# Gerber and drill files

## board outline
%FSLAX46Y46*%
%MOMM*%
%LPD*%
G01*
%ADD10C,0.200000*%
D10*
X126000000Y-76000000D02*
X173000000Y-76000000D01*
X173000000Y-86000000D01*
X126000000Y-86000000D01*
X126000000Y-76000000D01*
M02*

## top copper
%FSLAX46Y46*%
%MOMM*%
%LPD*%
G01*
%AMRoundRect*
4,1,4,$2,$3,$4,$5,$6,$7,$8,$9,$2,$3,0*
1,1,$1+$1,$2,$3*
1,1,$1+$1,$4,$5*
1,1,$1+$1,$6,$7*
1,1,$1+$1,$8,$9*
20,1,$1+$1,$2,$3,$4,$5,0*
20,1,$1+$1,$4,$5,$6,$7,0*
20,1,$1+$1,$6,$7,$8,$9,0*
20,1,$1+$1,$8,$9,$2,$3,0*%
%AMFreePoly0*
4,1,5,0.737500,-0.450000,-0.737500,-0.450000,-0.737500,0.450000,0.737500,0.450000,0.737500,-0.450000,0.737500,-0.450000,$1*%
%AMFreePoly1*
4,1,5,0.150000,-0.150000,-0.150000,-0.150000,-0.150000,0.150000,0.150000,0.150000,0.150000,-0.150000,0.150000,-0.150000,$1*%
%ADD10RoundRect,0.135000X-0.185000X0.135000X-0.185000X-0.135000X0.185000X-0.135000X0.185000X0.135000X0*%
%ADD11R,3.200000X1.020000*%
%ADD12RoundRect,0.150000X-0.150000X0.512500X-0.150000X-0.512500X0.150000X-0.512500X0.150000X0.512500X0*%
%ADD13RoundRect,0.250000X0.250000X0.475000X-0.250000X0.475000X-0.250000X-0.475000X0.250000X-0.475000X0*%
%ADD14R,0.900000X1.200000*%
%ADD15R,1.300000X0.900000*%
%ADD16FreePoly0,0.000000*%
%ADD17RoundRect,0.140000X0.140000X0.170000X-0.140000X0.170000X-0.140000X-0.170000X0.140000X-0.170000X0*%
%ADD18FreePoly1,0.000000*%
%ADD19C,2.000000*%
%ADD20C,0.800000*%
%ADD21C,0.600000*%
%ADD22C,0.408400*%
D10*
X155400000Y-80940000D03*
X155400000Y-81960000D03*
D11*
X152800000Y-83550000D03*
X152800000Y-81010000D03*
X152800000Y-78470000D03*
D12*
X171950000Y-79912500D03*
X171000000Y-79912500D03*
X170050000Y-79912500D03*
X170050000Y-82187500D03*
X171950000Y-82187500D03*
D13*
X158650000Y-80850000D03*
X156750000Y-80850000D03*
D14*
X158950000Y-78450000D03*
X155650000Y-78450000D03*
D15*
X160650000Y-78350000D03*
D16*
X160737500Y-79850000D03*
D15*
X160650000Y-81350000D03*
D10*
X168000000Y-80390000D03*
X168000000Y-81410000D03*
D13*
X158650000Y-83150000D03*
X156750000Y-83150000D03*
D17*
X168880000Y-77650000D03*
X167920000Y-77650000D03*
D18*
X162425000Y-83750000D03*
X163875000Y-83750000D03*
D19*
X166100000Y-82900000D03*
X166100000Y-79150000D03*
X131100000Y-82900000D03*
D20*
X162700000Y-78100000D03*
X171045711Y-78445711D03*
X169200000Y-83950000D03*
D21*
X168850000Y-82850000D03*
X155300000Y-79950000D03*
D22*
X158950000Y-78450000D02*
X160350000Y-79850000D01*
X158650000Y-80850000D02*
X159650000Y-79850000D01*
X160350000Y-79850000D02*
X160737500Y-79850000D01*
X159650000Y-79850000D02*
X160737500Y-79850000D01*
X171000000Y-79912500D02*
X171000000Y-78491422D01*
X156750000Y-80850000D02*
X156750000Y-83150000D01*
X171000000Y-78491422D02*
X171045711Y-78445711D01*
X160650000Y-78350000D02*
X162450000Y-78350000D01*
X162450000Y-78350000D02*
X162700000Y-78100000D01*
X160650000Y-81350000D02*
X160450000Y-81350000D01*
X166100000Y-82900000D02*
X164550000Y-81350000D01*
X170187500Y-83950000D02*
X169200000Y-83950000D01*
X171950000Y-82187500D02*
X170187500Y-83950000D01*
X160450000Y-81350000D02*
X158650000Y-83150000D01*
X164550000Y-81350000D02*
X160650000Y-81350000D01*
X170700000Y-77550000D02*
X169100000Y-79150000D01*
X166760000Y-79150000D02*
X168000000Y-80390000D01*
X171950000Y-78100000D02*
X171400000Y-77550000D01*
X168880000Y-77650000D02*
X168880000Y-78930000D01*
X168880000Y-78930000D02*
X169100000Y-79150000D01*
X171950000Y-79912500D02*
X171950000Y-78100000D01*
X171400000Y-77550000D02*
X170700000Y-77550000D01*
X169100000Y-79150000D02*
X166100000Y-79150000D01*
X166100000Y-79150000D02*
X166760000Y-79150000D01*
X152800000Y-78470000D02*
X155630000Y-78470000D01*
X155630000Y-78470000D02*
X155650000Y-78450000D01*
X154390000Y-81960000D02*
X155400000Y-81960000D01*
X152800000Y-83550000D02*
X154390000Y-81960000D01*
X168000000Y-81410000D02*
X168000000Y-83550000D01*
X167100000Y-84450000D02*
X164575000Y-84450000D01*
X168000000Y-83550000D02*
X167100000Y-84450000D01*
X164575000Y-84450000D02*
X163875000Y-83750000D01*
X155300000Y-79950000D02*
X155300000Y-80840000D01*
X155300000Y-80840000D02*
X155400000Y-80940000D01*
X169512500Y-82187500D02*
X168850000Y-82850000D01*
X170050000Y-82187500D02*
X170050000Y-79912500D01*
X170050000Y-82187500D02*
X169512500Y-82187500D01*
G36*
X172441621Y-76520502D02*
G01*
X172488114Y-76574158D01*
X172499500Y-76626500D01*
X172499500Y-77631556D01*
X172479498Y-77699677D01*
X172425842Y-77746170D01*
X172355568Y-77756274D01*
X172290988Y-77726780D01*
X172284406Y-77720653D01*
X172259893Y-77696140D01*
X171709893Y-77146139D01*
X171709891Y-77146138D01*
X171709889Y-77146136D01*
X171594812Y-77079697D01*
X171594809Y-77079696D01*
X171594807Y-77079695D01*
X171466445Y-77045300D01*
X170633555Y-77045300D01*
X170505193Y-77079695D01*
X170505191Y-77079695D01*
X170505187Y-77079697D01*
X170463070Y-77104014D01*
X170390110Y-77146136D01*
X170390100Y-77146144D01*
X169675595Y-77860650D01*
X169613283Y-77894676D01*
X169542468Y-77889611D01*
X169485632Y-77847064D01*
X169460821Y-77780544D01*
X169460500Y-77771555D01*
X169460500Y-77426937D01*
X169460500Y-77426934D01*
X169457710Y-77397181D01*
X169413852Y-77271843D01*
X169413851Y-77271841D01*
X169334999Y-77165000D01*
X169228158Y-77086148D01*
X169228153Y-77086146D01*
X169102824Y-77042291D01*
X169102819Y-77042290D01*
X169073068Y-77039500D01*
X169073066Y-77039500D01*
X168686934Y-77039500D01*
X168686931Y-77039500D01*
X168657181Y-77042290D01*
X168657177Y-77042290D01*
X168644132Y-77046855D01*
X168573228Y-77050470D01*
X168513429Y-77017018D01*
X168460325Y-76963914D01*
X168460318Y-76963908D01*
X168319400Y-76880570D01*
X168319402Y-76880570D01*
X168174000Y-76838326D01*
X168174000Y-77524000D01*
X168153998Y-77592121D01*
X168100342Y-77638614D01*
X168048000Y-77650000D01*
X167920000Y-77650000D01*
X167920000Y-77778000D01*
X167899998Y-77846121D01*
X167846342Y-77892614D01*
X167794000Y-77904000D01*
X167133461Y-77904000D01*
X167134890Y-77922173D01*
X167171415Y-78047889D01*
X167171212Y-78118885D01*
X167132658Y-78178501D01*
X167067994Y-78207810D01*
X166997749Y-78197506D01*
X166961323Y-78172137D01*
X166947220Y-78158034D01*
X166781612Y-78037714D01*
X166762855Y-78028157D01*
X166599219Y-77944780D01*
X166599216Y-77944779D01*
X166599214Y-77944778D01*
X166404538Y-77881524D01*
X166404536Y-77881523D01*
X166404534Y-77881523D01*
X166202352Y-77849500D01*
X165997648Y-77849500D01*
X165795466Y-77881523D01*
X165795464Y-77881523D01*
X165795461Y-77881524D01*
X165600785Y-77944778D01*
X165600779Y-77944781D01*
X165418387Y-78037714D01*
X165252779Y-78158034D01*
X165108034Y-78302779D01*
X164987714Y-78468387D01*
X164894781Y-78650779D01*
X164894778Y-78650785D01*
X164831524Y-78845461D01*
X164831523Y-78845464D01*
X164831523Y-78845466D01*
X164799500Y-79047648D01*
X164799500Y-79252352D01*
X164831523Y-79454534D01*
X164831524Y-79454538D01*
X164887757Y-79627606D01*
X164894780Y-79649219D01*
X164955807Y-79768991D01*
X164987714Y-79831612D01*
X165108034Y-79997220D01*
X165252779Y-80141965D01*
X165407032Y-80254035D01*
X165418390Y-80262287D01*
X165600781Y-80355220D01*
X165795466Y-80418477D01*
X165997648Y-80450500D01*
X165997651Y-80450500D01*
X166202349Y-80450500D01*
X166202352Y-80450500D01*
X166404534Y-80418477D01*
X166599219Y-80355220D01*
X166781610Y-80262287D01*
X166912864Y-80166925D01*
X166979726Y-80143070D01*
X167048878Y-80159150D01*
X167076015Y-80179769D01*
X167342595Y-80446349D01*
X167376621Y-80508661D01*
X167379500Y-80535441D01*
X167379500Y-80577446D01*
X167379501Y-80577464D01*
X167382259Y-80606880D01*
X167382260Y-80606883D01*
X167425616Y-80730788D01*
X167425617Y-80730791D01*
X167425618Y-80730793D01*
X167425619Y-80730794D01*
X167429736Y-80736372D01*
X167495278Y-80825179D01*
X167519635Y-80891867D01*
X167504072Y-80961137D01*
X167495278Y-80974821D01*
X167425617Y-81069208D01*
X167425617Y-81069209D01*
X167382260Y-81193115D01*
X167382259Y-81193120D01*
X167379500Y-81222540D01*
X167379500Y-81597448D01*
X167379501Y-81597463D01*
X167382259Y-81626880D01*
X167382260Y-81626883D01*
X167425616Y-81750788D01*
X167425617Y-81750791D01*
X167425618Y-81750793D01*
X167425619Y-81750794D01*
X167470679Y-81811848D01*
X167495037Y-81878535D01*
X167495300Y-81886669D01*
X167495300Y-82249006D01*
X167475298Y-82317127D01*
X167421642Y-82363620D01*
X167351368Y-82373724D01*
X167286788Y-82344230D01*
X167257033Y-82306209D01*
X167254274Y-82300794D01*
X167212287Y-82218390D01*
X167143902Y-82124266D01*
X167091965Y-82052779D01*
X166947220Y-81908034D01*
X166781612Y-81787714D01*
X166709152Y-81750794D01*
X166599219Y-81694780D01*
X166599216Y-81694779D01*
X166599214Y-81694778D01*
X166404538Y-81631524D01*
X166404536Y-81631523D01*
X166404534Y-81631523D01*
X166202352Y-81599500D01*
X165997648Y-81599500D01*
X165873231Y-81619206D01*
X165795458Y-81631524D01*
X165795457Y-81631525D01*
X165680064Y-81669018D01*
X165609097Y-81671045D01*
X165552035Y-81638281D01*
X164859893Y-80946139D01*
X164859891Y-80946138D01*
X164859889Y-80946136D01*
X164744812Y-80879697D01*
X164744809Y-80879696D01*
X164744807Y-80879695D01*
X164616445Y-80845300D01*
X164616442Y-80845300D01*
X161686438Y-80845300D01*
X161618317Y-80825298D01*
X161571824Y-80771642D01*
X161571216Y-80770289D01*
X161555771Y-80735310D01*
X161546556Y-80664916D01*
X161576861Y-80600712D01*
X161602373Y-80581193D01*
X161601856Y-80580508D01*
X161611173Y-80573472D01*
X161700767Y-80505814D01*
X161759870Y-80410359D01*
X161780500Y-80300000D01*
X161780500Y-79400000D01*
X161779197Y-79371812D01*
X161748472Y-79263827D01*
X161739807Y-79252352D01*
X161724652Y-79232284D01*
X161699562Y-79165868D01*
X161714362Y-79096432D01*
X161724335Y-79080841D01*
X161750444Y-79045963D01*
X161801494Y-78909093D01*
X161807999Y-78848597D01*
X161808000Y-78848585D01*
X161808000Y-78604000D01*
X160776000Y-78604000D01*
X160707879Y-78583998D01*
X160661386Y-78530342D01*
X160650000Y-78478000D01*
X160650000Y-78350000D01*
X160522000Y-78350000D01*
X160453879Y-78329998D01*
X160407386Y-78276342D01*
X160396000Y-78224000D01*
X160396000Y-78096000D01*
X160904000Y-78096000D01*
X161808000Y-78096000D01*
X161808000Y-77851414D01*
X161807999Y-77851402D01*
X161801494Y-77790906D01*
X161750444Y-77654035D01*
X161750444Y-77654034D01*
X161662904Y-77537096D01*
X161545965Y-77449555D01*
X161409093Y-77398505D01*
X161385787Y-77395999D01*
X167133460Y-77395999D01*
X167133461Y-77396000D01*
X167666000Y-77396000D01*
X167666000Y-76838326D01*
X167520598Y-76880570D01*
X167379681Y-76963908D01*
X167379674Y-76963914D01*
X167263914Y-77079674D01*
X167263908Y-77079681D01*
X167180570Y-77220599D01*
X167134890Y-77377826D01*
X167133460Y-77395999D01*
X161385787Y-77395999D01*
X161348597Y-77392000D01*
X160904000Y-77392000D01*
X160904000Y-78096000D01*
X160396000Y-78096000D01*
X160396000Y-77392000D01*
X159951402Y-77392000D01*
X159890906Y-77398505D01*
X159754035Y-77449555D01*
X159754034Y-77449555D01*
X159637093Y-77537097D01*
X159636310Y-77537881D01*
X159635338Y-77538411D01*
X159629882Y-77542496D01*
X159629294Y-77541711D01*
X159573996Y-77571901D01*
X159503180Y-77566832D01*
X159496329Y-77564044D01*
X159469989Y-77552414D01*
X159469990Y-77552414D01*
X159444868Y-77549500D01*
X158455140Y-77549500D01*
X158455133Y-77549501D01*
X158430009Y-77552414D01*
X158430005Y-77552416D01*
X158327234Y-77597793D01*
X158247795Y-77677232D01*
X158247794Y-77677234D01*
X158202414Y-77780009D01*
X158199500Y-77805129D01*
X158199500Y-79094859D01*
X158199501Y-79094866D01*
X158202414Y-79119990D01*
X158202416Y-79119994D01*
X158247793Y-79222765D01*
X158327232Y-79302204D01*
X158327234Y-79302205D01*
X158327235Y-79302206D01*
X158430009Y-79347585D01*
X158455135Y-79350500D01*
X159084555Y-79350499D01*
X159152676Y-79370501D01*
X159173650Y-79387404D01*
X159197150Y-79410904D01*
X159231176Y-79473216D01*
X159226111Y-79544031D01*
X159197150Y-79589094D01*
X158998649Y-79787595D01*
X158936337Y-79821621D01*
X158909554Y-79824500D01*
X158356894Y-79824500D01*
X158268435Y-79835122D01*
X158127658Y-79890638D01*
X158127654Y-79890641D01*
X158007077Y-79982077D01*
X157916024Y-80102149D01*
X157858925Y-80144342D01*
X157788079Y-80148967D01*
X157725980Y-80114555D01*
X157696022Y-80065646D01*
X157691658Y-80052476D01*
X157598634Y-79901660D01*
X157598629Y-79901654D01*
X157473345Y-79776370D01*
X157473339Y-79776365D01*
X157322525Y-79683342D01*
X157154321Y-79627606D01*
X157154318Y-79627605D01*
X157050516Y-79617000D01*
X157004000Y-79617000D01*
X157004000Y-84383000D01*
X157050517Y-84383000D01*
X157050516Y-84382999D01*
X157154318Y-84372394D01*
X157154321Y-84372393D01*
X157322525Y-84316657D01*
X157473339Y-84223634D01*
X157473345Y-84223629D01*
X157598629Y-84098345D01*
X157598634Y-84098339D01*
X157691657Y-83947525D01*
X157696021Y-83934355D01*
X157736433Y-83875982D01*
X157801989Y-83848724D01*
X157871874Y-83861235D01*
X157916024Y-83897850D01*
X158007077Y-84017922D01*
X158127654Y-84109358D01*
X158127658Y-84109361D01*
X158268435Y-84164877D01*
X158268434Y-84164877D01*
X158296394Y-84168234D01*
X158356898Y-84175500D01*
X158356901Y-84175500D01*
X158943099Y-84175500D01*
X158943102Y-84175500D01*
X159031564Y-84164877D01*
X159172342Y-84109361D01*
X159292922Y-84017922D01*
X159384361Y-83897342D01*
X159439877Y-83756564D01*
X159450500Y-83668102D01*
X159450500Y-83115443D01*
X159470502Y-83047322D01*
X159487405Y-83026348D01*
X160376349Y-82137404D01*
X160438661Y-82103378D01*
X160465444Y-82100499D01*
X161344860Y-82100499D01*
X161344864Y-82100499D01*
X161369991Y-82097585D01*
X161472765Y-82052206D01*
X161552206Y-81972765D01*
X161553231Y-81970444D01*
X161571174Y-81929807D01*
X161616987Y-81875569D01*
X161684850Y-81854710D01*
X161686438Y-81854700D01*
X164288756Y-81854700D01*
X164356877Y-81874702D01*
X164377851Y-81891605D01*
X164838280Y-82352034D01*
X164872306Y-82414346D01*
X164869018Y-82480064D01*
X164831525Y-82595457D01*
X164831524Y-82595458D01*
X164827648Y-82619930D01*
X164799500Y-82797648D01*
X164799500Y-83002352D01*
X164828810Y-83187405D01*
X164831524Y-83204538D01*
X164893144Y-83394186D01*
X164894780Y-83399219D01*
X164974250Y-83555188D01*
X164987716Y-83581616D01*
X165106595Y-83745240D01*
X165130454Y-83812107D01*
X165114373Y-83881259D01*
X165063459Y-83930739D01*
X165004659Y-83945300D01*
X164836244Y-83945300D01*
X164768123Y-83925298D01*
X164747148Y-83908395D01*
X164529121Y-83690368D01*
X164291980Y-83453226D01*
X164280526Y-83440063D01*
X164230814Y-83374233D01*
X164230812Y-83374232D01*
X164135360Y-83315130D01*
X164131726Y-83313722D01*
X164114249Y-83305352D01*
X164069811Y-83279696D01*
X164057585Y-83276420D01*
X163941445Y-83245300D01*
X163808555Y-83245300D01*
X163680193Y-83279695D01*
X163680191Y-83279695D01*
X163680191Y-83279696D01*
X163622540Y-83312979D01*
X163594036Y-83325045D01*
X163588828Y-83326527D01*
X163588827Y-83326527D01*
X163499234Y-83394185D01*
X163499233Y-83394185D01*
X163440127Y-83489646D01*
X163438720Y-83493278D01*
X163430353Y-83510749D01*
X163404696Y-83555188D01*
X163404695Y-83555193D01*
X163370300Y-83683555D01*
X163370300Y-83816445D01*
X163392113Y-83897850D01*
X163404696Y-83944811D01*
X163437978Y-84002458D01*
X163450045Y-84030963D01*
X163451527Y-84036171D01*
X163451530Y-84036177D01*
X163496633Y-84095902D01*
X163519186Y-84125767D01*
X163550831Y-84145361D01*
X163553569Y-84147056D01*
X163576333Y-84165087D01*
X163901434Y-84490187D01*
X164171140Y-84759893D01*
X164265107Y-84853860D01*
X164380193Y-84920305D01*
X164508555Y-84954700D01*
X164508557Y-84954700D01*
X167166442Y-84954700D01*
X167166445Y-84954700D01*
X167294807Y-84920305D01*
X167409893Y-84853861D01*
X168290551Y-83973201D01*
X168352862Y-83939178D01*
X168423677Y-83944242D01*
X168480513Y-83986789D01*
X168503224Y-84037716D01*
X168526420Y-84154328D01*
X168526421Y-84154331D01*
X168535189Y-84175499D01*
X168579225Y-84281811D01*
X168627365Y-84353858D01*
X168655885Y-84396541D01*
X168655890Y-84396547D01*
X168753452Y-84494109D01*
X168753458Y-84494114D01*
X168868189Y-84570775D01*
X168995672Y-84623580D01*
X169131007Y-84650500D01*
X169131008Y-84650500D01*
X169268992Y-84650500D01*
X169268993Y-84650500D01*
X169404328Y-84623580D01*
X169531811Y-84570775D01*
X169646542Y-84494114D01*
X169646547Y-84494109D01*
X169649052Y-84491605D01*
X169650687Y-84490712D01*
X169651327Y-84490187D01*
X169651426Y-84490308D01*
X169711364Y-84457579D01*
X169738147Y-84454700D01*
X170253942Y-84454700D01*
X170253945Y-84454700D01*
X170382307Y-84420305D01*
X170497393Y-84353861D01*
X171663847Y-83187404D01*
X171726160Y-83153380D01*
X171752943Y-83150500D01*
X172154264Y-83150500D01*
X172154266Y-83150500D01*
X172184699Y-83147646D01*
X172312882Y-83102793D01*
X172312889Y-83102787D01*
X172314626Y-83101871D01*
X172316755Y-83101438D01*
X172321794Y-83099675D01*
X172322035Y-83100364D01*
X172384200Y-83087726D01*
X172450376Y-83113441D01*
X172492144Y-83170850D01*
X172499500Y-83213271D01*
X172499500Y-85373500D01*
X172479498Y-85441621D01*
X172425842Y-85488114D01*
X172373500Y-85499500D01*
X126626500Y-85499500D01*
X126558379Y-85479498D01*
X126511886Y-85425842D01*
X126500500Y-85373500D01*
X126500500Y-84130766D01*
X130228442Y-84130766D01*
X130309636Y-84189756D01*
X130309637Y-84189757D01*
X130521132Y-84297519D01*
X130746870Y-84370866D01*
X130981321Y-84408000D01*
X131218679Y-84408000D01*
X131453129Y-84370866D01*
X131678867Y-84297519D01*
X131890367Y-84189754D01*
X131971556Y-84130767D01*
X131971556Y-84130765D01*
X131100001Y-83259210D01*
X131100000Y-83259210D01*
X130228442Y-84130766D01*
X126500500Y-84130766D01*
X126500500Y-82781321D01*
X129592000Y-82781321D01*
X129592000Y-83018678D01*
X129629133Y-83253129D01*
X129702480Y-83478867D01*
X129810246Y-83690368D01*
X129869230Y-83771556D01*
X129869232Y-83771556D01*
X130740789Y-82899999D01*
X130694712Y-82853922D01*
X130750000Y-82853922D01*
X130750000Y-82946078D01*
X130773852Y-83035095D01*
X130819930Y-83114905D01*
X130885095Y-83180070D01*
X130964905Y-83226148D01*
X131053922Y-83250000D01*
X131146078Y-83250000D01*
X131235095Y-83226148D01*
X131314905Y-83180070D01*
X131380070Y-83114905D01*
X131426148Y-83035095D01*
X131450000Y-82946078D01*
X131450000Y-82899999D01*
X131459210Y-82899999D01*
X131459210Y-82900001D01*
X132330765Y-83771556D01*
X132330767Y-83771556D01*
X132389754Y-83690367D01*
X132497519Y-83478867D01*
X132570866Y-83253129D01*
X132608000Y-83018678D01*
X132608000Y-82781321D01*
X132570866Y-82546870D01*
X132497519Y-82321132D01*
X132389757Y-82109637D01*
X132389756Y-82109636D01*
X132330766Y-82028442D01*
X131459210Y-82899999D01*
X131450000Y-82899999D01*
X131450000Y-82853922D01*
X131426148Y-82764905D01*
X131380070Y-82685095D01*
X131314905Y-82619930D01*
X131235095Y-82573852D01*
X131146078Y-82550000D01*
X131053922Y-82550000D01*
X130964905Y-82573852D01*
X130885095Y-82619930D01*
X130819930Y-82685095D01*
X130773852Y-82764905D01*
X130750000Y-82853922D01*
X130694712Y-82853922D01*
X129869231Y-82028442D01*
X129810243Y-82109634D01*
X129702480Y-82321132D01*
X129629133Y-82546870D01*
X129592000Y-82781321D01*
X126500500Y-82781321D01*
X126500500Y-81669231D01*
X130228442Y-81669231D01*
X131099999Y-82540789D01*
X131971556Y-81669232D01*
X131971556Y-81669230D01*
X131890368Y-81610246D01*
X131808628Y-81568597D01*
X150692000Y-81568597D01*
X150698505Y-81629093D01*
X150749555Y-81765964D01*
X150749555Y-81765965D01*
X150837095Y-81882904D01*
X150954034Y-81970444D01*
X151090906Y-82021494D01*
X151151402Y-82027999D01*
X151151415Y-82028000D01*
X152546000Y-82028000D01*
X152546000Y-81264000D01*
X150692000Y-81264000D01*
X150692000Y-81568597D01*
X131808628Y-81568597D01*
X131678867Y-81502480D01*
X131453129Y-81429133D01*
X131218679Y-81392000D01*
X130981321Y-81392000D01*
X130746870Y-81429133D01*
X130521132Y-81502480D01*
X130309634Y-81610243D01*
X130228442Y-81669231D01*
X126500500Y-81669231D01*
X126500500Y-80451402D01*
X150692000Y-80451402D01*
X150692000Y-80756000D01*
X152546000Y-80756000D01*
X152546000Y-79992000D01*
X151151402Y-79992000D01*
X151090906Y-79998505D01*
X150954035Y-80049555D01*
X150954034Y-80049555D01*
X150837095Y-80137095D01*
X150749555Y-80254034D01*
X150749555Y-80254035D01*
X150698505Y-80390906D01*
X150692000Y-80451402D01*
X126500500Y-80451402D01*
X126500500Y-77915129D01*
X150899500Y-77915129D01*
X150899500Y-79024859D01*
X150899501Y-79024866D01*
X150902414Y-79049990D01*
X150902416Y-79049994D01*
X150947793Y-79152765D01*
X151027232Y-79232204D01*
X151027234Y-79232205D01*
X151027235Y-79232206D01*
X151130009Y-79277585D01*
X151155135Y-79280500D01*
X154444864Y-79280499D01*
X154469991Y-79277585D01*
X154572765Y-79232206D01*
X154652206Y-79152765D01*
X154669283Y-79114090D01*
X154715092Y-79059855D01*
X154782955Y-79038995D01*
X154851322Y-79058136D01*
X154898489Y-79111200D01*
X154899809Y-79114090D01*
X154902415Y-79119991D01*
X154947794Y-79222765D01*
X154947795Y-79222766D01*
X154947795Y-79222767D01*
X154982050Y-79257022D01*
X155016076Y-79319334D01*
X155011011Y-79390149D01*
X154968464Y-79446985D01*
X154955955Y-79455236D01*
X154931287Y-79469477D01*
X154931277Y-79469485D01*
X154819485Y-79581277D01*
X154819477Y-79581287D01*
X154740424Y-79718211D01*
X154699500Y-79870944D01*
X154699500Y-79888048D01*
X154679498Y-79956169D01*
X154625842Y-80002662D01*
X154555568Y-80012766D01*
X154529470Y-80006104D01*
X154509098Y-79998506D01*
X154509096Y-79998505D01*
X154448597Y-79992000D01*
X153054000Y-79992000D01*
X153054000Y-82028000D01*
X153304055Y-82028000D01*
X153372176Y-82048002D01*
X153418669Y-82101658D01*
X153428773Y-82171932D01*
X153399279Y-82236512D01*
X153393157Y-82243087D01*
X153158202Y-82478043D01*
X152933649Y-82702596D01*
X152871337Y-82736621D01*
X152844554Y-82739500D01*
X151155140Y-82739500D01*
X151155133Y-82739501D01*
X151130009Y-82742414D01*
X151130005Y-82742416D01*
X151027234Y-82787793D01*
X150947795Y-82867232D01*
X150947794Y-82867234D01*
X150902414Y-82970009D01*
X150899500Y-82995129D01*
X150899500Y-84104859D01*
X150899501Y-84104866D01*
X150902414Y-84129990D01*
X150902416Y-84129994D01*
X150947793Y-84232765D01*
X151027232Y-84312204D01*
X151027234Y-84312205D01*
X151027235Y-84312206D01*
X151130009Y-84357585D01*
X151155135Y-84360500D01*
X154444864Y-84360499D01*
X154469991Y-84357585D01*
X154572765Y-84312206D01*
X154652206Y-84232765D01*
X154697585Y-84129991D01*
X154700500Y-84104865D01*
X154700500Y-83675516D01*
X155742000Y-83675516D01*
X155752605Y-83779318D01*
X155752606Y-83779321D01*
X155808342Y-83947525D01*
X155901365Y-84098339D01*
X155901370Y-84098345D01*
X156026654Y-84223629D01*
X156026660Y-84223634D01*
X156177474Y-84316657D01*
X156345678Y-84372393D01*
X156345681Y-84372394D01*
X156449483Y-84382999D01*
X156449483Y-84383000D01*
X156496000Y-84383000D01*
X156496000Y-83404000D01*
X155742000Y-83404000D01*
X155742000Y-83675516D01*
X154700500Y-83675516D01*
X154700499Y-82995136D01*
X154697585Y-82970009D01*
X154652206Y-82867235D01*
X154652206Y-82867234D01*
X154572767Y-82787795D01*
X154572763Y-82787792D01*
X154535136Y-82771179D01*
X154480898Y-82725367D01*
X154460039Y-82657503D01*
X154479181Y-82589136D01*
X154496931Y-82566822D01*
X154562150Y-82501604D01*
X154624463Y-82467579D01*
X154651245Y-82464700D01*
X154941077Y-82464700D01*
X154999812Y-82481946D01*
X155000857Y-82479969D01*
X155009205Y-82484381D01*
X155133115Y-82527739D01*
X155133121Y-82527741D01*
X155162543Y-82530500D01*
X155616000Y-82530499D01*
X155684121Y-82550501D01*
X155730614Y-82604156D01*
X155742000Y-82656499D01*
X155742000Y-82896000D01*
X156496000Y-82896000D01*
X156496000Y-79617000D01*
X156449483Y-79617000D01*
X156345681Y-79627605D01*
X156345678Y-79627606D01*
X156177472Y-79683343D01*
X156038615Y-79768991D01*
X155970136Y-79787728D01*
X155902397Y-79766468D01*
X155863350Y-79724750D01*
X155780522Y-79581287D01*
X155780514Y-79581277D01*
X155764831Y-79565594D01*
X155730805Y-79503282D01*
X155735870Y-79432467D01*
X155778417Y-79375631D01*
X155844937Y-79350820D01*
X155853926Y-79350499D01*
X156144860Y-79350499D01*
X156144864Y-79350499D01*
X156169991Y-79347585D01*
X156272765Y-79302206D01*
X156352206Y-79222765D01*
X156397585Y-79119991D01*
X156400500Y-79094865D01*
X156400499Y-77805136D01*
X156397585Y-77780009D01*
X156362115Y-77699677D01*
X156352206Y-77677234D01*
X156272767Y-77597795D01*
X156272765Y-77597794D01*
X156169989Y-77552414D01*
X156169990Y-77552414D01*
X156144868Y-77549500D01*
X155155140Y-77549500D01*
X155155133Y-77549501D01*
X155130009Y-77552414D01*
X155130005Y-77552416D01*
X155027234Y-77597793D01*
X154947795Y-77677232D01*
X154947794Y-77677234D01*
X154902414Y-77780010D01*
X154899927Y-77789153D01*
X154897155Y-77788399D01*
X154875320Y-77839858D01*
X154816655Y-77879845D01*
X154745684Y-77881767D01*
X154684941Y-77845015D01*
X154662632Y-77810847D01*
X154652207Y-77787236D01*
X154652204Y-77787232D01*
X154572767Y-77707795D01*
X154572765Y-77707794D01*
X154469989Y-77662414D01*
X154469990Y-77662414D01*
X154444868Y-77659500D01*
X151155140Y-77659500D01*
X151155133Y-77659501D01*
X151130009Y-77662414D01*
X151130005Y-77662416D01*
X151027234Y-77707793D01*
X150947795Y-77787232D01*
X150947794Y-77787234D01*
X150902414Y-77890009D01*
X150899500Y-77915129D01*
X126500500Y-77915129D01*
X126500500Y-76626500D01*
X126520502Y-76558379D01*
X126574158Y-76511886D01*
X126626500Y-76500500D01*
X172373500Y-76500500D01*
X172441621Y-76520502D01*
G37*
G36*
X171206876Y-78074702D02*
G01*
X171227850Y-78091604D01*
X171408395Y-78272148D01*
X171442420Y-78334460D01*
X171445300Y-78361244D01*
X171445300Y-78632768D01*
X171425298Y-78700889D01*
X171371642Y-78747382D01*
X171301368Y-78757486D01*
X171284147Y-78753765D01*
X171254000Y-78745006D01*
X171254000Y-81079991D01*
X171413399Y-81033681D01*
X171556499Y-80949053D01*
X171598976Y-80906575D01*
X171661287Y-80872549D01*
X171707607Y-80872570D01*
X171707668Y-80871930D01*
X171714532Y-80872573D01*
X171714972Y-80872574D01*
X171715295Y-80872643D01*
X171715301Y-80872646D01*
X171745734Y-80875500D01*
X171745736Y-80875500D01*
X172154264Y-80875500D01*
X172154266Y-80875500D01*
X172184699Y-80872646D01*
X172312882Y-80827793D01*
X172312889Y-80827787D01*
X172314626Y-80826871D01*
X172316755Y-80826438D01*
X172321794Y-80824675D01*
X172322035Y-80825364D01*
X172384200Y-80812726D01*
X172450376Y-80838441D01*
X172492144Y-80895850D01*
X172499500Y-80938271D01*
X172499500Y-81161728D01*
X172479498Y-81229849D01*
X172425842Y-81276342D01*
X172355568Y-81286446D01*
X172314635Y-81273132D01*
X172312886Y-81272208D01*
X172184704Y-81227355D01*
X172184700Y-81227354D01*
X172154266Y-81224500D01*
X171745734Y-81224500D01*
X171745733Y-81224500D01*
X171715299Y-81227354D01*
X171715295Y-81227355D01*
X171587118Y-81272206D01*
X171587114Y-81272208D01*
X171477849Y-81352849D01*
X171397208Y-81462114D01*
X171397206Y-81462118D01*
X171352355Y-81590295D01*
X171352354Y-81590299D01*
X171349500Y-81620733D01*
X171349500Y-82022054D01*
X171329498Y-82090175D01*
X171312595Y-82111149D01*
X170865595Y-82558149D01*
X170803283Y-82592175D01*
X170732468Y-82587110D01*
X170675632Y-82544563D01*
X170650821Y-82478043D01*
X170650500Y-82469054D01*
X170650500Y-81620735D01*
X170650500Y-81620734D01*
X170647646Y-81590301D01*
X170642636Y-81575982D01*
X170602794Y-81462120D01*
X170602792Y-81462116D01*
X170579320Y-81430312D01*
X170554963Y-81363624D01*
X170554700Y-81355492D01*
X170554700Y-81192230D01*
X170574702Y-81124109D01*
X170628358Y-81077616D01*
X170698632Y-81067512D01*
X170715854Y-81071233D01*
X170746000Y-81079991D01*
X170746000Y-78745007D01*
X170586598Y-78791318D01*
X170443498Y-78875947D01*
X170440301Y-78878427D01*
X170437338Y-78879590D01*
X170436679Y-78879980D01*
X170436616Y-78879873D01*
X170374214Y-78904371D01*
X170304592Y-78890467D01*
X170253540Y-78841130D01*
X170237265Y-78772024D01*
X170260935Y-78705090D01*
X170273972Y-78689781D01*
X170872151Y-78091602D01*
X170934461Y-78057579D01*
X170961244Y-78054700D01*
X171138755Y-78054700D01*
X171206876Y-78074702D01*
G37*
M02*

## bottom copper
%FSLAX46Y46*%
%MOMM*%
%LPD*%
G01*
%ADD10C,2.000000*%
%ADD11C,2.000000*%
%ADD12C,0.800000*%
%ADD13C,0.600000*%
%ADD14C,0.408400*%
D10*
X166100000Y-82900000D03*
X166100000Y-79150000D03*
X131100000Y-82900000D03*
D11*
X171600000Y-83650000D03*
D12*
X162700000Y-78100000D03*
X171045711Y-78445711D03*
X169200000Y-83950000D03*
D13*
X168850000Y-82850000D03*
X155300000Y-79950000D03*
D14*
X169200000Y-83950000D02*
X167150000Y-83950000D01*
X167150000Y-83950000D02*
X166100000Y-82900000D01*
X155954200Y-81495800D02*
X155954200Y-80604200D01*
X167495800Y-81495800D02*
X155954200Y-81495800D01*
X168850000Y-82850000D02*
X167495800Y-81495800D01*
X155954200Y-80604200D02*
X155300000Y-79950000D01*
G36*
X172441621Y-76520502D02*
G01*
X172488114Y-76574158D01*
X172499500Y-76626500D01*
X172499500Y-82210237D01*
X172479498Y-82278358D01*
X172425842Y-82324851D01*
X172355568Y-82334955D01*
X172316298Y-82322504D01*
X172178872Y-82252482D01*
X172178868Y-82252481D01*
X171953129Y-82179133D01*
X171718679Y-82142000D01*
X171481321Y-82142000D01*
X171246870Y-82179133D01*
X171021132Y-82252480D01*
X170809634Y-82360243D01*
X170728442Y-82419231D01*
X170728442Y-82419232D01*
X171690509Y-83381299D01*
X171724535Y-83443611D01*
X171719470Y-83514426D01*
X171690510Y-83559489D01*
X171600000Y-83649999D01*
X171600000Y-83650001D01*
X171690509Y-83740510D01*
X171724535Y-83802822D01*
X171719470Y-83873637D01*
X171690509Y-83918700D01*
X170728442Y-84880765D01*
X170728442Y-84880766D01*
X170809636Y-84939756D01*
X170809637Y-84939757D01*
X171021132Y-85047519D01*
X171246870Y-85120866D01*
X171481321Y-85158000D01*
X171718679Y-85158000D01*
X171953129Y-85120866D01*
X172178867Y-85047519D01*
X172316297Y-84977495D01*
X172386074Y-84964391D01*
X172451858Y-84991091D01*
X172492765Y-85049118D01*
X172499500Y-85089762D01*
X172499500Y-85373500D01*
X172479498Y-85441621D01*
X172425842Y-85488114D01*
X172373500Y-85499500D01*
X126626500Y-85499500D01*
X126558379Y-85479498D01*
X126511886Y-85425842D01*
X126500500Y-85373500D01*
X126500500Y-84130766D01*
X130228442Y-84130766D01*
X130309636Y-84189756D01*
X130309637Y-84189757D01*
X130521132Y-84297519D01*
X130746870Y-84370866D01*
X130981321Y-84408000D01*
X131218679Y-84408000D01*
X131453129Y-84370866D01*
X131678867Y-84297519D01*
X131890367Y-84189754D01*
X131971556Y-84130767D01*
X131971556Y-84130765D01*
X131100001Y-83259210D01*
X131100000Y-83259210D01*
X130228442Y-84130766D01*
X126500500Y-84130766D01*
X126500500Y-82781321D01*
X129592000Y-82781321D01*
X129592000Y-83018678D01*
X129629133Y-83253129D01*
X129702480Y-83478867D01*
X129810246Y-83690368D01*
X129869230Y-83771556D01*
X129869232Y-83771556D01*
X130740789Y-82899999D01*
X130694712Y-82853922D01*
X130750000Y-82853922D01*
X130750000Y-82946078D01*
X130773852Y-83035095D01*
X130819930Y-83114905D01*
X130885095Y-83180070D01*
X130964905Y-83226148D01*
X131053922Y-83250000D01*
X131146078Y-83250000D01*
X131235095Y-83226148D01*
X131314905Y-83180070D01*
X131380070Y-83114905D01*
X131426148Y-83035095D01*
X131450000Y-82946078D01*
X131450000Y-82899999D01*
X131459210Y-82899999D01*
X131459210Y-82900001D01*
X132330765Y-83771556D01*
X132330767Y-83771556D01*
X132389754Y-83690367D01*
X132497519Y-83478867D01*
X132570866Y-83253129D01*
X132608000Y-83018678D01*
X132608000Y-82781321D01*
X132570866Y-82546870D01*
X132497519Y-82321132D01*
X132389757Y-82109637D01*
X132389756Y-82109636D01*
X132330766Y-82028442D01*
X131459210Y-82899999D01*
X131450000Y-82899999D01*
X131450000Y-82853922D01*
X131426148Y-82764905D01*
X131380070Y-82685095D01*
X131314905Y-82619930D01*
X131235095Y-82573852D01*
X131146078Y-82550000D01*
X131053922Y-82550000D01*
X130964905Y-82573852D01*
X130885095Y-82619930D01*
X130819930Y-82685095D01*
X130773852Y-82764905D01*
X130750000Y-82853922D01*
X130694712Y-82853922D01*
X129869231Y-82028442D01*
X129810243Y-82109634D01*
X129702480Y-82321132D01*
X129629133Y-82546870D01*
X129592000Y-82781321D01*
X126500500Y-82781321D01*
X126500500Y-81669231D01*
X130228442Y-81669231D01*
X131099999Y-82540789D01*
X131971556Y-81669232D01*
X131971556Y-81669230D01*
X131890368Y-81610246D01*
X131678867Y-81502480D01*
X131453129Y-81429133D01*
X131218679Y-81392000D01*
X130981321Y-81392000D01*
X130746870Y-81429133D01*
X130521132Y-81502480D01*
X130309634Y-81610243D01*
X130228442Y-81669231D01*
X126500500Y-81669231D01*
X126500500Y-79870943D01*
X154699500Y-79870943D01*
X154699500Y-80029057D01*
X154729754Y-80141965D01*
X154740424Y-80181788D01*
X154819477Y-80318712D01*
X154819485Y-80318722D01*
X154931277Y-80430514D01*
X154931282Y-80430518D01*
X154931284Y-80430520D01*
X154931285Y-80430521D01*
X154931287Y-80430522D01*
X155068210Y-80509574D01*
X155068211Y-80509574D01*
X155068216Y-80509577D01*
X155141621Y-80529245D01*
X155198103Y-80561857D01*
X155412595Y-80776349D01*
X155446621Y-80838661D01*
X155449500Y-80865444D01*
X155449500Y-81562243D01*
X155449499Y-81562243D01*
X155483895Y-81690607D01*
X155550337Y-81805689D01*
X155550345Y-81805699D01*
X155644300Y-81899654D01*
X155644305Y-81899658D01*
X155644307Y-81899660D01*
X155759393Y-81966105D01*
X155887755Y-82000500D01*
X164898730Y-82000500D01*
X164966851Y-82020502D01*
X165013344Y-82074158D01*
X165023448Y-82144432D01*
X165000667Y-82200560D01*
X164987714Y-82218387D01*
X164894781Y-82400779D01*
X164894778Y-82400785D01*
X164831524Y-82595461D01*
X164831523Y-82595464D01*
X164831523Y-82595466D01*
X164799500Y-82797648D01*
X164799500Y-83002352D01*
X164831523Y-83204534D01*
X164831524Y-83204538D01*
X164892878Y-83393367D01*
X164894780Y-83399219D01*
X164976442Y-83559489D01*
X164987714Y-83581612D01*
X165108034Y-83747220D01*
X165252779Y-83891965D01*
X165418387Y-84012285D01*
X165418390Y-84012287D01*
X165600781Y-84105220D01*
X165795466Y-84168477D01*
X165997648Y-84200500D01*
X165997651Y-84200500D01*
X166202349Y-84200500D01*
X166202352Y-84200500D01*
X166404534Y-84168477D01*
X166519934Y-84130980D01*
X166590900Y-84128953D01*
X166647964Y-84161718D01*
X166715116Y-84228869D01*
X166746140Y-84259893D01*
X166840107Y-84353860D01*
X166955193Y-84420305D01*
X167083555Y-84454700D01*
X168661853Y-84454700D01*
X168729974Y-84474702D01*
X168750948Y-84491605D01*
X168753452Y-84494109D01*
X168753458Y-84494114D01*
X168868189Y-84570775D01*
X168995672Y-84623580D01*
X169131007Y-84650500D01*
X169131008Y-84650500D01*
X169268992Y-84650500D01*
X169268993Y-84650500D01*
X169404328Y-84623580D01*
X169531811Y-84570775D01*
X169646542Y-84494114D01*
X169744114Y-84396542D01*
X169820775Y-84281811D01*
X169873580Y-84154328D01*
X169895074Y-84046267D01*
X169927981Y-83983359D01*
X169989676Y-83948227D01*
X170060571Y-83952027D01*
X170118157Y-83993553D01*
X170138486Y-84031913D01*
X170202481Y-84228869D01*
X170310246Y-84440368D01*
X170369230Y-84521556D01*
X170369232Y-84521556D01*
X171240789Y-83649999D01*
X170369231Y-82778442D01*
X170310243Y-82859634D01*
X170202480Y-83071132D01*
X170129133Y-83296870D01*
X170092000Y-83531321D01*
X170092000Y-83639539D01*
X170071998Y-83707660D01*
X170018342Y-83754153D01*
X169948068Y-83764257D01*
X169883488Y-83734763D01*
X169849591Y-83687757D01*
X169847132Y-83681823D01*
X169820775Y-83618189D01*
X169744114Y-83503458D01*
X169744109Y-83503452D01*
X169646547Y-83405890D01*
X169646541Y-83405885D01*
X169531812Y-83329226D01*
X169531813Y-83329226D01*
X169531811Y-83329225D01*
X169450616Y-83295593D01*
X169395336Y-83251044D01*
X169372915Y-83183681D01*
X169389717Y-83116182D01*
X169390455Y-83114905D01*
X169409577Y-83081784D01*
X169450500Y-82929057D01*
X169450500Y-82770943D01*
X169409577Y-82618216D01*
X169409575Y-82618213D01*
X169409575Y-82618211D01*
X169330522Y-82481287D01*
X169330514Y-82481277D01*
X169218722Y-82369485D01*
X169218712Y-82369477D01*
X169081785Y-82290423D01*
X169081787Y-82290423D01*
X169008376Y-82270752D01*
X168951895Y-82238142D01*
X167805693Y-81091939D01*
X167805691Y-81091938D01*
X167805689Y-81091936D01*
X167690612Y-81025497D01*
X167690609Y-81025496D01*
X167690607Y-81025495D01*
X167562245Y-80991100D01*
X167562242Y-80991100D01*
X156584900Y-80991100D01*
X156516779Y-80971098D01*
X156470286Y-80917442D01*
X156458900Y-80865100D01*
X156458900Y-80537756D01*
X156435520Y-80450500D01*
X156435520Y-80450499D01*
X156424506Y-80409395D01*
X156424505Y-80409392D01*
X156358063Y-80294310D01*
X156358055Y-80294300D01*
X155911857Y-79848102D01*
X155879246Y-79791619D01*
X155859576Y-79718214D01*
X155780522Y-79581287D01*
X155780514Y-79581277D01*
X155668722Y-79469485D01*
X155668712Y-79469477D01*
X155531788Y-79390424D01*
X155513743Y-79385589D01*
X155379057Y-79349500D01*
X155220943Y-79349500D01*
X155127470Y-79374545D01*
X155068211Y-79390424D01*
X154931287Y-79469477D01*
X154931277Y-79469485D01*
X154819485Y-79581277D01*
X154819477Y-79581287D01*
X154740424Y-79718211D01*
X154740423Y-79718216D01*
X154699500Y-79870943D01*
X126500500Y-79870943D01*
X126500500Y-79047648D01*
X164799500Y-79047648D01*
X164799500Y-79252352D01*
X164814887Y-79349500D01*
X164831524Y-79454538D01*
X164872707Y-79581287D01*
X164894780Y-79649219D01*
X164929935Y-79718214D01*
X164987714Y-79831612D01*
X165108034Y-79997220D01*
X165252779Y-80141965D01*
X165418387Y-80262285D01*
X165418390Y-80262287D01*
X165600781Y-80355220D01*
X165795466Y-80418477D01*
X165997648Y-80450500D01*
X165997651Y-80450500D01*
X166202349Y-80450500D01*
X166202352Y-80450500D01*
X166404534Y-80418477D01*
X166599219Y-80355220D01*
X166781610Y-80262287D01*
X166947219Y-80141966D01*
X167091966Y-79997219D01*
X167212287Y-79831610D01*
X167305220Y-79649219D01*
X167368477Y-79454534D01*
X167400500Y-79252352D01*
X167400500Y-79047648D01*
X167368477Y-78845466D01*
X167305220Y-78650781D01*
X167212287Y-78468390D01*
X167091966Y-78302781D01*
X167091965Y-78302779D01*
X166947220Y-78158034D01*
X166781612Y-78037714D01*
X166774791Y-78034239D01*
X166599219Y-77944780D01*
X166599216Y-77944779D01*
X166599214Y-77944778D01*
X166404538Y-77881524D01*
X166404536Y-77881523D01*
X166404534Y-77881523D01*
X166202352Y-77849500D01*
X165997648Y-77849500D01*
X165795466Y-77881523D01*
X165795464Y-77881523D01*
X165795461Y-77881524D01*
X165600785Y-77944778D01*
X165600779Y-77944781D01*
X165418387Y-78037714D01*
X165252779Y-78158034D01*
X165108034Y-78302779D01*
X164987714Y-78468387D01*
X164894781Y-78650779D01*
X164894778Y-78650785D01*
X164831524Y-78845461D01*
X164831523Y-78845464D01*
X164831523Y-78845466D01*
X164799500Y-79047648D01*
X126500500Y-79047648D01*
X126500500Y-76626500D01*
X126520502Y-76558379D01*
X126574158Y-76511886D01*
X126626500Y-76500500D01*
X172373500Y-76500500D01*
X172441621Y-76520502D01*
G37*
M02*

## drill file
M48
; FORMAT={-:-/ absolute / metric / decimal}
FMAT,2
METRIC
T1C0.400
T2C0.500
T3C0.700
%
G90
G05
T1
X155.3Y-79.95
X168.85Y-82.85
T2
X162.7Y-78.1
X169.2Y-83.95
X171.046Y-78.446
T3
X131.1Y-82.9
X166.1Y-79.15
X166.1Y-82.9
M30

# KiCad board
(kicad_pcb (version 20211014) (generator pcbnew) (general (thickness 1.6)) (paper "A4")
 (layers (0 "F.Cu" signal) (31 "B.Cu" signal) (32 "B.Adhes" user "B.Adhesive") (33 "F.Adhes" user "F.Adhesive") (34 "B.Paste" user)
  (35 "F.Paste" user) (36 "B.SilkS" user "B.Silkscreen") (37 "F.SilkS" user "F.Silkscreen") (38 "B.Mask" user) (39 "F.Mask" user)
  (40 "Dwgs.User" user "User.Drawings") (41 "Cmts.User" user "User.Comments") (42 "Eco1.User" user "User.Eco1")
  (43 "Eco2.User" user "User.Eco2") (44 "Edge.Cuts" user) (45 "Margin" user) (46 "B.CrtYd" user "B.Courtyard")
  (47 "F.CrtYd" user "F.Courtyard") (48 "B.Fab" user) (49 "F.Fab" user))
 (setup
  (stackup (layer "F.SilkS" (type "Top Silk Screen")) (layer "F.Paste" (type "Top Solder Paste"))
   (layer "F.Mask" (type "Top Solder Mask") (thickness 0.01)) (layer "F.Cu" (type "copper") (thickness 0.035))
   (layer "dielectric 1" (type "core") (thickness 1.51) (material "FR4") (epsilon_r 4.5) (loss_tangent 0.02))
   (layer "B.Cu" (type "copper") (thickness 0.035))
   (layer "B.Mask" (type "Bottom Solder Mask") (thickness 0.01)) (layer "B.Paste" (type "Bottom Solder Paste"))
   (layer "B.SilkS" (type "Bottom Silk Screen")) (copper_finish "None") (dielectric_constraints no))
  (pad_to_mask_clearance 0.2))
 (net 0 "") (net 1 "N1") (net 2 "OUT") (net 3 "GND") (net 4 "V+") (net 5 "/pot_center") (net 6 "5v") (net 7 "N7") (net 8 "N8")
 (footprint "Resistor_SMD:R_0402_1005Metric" (layer "F.Cu") (at 155.4 81.45 -90)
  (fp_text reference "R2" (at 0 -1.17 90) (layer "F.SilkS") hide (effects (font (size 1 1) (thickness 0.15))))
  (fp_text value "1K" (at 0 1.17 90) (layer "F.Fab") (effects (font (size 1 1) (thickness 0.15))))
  (pad "1" smd roundrect (at -0.51 0 270) (size 0.54 0.64) (layers "F.Cu" "F.Paste" "F.Mask") (roundrect_rratio 0.25) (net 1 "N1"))
  (pad "2" smd roundrect (at 0.51 0 270) (size 0.54 0.64) (layers "F.Cu" "F.Paste" "F.Mask") (roundrect_rratio 0.25) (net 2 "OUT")))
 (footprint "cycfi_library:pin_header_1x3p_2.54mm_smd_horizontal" (layer "F.Cu") (at 152.8 81.01 180)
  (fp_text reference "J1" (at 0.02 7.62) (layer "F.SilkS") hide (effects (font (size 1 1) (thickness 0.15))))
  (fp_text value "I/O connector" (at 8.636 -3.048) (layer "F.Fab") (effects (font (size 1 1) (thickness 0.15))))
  (pad "1" smd rect (at 0 -2.54 180) (size 3.2 1.02) (layers "F.Cu" "F.Paste" "F.Mask") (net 2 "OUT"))
  (pad "2" smd rect (at 0 0 180) (size 3.2 1.02) (layers "F.Cu" "F.Paste" "F.Mask") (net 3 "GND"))
  (pad "3" smd rect (at 0 2.54 180) (size 3.2 1.02) (layers "F.Cu" "F.Paste" "F.Mask") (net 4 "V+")))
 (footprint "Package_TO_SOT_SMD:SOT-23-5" (layer "F.Cu") (at 171 81.05 -90)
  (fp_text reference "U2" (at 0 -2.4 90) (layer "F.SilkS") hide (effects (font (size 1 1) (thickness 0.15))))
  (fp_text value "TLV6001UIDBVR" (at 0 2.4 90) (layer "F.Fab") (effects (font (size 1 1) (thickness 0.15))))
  (pad "1" smd roundrect (at -1.1375 -0.95 270) (size 1.325 0.6) (layers "F.Cu" "F.Paste" "F.Mask") (roundrect_rratio 0.25)
   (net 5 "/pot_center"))
  (pad "2" smd roundrect (at -1.1375 0 270) (size 1.325 0.6) (layers "F.Cu" "F.Paste" "F.Mask") (roundrect_rratio 0.25) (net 3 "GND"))
  (pad "3" smd roundrect (at -1.1375 0.95 270) (size 1.325 0.6) (layers "F.Cu" "F.Paste" "F.Mask") (roundrect_rratio 0.25) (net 1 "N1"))
  (pad "4" smd roundrect (at 1.1375 0.95 270) (size 1.325 0.6) (layers "F.Cu" "F.Paste" "F.Mask") (roundrect_rratio 0.25) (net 1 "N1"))
  (pad "5" smd roundrect (at 1.1375 -0.95 270) (size 1.325 0.6) (layers "F.Cu" "F.Paste" "F.Mask") (roundrect_rratio 0.25) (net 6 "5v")))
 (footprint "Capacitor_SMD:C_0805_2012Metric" (layer "F.Cu") (at 157.7 80.85 180)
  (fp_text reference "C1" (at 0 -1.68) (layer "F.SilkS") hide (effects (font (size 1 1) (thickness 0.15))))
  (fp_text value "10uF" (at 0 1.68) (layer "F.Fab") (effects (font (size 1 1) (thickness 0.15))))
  (pad "1" smd roundrect (at -0.95 0 180) (size 1 1.45) (layers "F.Cu" "F.Paste" "F.Mask") (roundrect_rratio 0.25) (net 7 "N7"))
  (pad "2" smd roundrect (at 0.95 0 180) (size 1 1.45) (layers "F.Cu" "F.Paste" "F.Mask") (roundrect_rratio 0.25) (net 3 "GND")))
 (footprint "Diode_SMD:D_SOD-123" (layer "F.Cu") (at 157.3 78.45 180)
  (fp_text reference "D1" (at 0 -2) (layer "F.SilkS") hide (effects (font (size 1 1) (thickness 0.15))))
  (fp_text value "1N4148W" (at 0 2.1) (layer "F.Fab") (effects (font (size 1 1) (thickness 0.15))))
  (pad "1" smd rect (at -1.65 0 180) (size 0.9 1.2) (layers "F.Cu" "F.Paste" "F.Mask") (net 7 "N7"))
  (pad "2" smd rect (at 1.65 0 180) (size 0.9 1.2) (layers "F.Cu" "F.Paste" "F.Mask") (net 4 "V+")))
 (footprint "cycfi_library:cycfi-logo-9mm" (layer "F.Cu") (at 141.5 82.85)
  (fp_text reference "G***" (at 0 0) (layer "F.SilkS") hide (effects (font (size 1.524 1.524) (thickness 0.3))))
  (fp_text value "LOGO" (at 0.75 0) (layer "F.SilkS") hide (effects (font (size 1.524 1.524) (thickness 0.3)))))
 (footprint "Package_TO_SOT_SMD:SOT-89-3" (layer "F.Cu") (at 162.3 79.85)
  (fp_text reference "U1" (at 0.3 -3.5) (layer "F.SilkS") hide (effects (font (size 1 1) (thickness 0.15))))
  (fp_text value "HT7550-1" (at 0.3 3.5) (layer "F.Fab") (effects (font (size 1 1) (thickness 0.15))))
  (pad "1" smd rect (at -1.65 -1.5) (size 1.3 0.9) (layers "F.Cu" "F.Paste" "F.Mask") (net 3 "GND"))
  (pad "2" smd custom (at -1.5625 0) (size 1.475 0.9) (layers "F.Cu" "F.Paste" "F.Mask") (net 7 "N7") (zone_connect 2)
   (options (clearance outline) (anchor rect)) (primitives))
  (pad "3" smd rect (at -1.65 1.5) (size 1.3 0.9) (layers "F.Cu" "F.Paste" "F.Mask") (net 6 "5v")))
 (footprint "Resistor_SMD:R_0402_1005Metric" (layer "F.Cu") (at 168 80.9 -90)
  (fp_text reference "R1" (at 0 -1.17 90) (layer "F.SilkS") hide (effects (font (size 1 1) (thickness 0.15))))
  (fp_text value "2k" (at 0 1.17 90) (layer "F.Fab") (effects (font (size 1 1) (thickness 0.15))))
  (pad "1" smd roundrect (at -0.51 0 270) (size 0.54 0.64) (layers "F.Cu" "F.Paste" "F.Mask") (roundrect_rratio 0.25) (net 5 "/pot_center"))
  (pad "2" smd roundrect (at 0.51 0 270) (size 0.54 0.64) (layers "F.Cu" "F.Paste" "F.Mask") (roundrect_rratio 0.25) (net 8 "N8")))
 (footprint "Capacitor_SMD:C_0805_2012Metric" (layer "F.Cu") (at 157.7 83.15 180)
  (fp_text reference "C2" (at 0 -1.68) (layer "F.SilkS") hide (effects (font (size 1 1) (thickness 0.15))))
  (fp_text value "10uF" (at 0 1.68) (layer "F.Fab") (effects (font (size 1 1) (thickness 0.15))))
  (pad "1" smd roundrect (at -0.95 0 180) (size 1 1.45) (layers "F.Cu" "F.Paste" "F.Mask") (roundrect_rratio 0.25) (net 6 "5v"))
  (pad "2" smd roundrect (at 0.95 0 180) (size 1 1.45) (layers "F.Cu" "F.Paste" "F.Mask") (roundrect_rratio 0.25) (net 3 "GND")))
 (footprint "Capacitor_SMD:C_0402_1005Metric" (layer "F.Cu") (at 168.4 77.65 180)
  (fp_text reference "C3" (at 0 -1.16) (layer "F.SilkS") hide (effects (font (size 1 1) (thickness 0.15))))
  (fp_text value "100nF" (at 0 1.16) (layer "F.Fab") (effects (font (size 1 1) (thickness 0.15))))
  (pad "1" smd roundrect (at -0.48 0 180) (size 0.56 0.62) (layers "F.Cu" "F.Paste" "F.Mask") (roundrect_rratio 0.25) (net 5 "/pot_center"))
  (pad "2" smd roundrect (at 0.48 0 180) (size 0.56 0.62) (layers "F.Cu" "F.Paste" "F.Mask") (roundrect_rratio 0.25) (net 3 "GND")))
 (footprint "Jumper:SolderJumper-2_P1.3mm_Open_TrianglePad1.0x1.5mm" (layer "F.Cu") (at 163.15 83.75)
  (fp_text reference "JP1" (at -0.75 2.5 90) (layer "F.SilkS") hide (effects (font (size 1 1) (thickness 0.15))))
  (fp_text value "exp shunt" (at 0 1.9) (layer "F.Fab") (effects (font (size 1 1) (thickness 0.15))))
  (pad "1" smd custom (at -0.725 0) (size 0.3 0.3) (layers "F.Cu" "F.Mask") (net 3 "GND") (zone_connect 2)
   (options (clearance outline) (anchor rect)) (primitives))
  (pad "2" smd custom (at 0.725 0) (size 0.3 0.3) (layers "F.Cu" "F.Mask") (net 8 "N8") (zone_connect 2)
   (options (clearance outline) (anchor rect)) (primitives)))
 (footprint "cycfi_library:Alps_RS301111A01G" (layer "B.Cu") (at 148.6 81.025 180)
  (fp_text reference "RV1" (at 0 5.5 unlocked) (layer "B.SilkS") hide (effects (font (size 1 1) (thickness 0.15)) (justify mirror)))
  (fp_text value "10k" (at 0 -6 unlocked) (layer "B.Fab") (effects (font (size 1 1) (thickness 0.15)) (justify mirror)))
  (pad "1" thru_hole circle (at -17.5 -1.875 180) (size 2 2) (drill 0.7) (layers *.Cu *.Mask) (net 6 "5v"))
  (pad "2" thru_hole circle (at -17.5 1.875 180) (size 2 2) (drill 0.7) (layers *.Cu *.Mask) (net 5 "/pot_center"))
  (pad "3" thru_hole circle (at 17.5 -1.875 180) (size 2 2) (drill 0.7) (layers *.Cu *.Mask) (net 3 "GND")))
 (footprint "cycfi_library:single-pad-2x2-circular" (layer "B.Cu") (at 171.6 83.65 180)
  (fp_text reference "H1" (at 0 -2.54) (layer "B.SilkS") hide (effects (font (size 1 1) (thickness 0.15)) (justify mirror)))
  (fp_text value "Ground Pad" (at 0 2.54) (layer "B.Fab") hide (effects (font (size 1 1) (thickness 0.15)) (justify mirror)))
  (pad "1" smd circle (at 0 0 180) (size 2 2) (layers "B.Cu" "B.Paste" "B.Mask") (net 3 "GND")))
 (gr_rect (start 126 76) (end 173 86) (layer "Edge.Cuts") (width 0.2) (fill none))
 (segment (start 158.95 78.45) (end 160.35 79.85) (width 0.4084) (layer "F.Cu") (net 7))
 (segment (start 158.65 80.85) (end 159.65 79.85) (width 0.4084) (layer "F.Cu") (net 7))
 (segment (start 160.35 79.85) (end 160.7375 79.85) (width 0.4084) (layer "F.Cu") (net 7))
 (segment (start 159.65 79.85) (end 160.7375 79.85) (width 0.4084) (layer "F.Cu") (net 7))
 (segment (start 171 79.9125) (end 171 78.491422) (width 0.4084) (layer "F.Cu") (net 3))
 (segment (start 156.75 80.85) (end 156.75 83.15) (width 0.4084) (layer "F.Cu") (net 3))
 (segment (start 171 78.491422) (end 171.045711 78.445711) (width 0.4084) (layer "F.Cu") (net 3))
 (segment (start 160.65 78.35) (end 162.45 78.35) (width 0.4084) (layer "F.Cu") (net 3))
 (segment (start 162.45 78.35) (end 162.7 78.1) (width 0.4084) (layer "F.Cu") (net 3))
 (via (at 162.7 78.1) (size 0.8) (drill 0.5) (layers "F.Cu" "B.Cu") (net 3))
 (via (at 171.045711 78.445711) (size 0.8) (drill 0.5) (layers "F.Cu" "B.Cu") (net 3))
 (segment (start 160.65 81.35) (end 160.45 81.35) (width 0.4084) (layer "F.Cu") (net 6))
 (segment (start 166.1 82.9) (end 164.55 81.35) (width 0.4084) (layer "F.Cu") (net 6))
 (segment (start 170.1875 83.95) (end 169.2 83.95) (width 0.4084) (layer "F.Cu") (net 6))
 (segment (start 171.95 82.1875) (end 170.1875 83.95) (width 0.4084) (layer "F.Cu") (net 6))
 (segment (start 160.45 81.35) (end 158.65 83.15) (width 0.4084) (layer "F.Cu") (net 6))
 (segment (start 164.55 81.35) (end 160.65 81.35) (width 0.4084) (layer "F.Cu") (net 6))
 (via (at 169.2 83.95) (size 0.8) (drill 0.5) (layers "F.Cu" "B.Cu") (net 6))
 (segment (start 169.2 83.95) (end 167.15 83.95) (width 0.4084) (layer "B.Cu") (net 6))
 (segment (start 167.15 83.95) (end 166.1 82.9) (width 0.4084) (layer "B.Cu") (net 6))
 (segment (start 170.7 77.55) (end 169.1 79.15) (width 0.4084) (layer "F.Cu") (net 5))
 (segment (start 166.76 79.15) (end 168 80.39) (width 0.4084) (layer "F.Cu") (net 5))
 (segment (start 171.95 78.1) (end 171.4 77.55) (width 0.4084) (layer "F.Cu") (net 5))
 (segment (start 168.88 77.65) (end 168.88 78.93) (width 0.4084) (layer "F.Cu") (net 5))
 (segment (start 168.88 78.93) (end 169.1 79.15) (width 0.4084) (layer "F.Cu") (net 5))
 (segment (start 171.95 79.9125) (end 171.95 78.1) (width 0.4084) (layer "F.Cu") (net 5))
 (segment (start 171.4 77.55) (end 170.7 77.55) (width 0.4084) (layer "F.Cu") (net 5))
 (segment (start 169.1 79.15) (end 166.1 79.15) (width 0.4084) (layer "F.Cu") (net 5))
 (segment (start 166.1 79.15) (end 166.76 79.15) (width 0.4084) (layer "F.Cu") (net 5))
 (segment (start 152.8 78.47) (end 155.63 78.47) (width 0.4084) (layer "F.Cu") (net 4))
 (segment (start 155.63 78.47) (end 155.65 78.45) (width 0.4084) (layer "F.Cu") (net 4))
 (segment (start 154.39 81.96) (end 155.4 81.96) (width 0.4084) (layer "F.Cu") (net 2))
 (segment (start 152.8 83.55) (end 154.39 81.96) (width 0.4084) (layer "F.Cu") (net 2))
 (segment (start 168 81.41) (end 168 83.55) (width 0.4084) (layer "F.Cu") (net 8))
 (segment (start 167.1 84.45) (end 164.575 84.45) (width 0.4084) (layer "F.Cu") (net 8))
 (segment (start 168 83.55) (end 167.1 84.45) (width 0.4084) (layer "F.Cu") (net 8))
 (segment (start 164.575 84.45) (end 163.875 83.75) (width 0.4084) (layer "F.Cu") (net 8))
 (segment (start 155.3 79.95) (end 155.3 80.84) (width 0.4084) (layer "F.Cu") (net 1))
 (segment (start 155.3 80.84) (end 155.4 80.94) (width 0.4084) (layer "F.Cu") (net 1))
 (segment (start 169.5125 82.1875) (end 168.85 82.85) (width 0.4084) (layer "F.Cu") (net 1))
 (segment (start 170.05 82.1875) (end 170.05 79.9125) (width 0.4084) (layer "F.Cu") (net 1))
 (segment (start 170.05 82.1875) (end 169.5125 82.1875) (width 0.4084) (layer "F.Cu") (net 1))
 (via (at 168.85 82.85) (size 0.6) (drill 0.4) (layers "F.Cu" "B.Cu") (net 1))
 (via (at 155.3 79.95) (size 0.6) (drill 0.4) (layers "F.Cu" "B.Cu") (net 1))
 (segment (start 155.9542 81.4958) (end 155.9542 80.6042) (width 0.4084) (layer "B.Cu") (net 1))
 (segment (start 167.4958 81.4958) (end 155.9542 81.4958) (width 0.4084) (layer "B.Cu") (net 1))
 (segment (start 168.85 82.85) (end 167.4958 81.4958) (width 0.4084) (layer "B.Cu") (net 1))
 (segment (start 155.9542 80.6042) (end 155.3 79.95) (width 0.4084) (layer "B.Cu") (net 1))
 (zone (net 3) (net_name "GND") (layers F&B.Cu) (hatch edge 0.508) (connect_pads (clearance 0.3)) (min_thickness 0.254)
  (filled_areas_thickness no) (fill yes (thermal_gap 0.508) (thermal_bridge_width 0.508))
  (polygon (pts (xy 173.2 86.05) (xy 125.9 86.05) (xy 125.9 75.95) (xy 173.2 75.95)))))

